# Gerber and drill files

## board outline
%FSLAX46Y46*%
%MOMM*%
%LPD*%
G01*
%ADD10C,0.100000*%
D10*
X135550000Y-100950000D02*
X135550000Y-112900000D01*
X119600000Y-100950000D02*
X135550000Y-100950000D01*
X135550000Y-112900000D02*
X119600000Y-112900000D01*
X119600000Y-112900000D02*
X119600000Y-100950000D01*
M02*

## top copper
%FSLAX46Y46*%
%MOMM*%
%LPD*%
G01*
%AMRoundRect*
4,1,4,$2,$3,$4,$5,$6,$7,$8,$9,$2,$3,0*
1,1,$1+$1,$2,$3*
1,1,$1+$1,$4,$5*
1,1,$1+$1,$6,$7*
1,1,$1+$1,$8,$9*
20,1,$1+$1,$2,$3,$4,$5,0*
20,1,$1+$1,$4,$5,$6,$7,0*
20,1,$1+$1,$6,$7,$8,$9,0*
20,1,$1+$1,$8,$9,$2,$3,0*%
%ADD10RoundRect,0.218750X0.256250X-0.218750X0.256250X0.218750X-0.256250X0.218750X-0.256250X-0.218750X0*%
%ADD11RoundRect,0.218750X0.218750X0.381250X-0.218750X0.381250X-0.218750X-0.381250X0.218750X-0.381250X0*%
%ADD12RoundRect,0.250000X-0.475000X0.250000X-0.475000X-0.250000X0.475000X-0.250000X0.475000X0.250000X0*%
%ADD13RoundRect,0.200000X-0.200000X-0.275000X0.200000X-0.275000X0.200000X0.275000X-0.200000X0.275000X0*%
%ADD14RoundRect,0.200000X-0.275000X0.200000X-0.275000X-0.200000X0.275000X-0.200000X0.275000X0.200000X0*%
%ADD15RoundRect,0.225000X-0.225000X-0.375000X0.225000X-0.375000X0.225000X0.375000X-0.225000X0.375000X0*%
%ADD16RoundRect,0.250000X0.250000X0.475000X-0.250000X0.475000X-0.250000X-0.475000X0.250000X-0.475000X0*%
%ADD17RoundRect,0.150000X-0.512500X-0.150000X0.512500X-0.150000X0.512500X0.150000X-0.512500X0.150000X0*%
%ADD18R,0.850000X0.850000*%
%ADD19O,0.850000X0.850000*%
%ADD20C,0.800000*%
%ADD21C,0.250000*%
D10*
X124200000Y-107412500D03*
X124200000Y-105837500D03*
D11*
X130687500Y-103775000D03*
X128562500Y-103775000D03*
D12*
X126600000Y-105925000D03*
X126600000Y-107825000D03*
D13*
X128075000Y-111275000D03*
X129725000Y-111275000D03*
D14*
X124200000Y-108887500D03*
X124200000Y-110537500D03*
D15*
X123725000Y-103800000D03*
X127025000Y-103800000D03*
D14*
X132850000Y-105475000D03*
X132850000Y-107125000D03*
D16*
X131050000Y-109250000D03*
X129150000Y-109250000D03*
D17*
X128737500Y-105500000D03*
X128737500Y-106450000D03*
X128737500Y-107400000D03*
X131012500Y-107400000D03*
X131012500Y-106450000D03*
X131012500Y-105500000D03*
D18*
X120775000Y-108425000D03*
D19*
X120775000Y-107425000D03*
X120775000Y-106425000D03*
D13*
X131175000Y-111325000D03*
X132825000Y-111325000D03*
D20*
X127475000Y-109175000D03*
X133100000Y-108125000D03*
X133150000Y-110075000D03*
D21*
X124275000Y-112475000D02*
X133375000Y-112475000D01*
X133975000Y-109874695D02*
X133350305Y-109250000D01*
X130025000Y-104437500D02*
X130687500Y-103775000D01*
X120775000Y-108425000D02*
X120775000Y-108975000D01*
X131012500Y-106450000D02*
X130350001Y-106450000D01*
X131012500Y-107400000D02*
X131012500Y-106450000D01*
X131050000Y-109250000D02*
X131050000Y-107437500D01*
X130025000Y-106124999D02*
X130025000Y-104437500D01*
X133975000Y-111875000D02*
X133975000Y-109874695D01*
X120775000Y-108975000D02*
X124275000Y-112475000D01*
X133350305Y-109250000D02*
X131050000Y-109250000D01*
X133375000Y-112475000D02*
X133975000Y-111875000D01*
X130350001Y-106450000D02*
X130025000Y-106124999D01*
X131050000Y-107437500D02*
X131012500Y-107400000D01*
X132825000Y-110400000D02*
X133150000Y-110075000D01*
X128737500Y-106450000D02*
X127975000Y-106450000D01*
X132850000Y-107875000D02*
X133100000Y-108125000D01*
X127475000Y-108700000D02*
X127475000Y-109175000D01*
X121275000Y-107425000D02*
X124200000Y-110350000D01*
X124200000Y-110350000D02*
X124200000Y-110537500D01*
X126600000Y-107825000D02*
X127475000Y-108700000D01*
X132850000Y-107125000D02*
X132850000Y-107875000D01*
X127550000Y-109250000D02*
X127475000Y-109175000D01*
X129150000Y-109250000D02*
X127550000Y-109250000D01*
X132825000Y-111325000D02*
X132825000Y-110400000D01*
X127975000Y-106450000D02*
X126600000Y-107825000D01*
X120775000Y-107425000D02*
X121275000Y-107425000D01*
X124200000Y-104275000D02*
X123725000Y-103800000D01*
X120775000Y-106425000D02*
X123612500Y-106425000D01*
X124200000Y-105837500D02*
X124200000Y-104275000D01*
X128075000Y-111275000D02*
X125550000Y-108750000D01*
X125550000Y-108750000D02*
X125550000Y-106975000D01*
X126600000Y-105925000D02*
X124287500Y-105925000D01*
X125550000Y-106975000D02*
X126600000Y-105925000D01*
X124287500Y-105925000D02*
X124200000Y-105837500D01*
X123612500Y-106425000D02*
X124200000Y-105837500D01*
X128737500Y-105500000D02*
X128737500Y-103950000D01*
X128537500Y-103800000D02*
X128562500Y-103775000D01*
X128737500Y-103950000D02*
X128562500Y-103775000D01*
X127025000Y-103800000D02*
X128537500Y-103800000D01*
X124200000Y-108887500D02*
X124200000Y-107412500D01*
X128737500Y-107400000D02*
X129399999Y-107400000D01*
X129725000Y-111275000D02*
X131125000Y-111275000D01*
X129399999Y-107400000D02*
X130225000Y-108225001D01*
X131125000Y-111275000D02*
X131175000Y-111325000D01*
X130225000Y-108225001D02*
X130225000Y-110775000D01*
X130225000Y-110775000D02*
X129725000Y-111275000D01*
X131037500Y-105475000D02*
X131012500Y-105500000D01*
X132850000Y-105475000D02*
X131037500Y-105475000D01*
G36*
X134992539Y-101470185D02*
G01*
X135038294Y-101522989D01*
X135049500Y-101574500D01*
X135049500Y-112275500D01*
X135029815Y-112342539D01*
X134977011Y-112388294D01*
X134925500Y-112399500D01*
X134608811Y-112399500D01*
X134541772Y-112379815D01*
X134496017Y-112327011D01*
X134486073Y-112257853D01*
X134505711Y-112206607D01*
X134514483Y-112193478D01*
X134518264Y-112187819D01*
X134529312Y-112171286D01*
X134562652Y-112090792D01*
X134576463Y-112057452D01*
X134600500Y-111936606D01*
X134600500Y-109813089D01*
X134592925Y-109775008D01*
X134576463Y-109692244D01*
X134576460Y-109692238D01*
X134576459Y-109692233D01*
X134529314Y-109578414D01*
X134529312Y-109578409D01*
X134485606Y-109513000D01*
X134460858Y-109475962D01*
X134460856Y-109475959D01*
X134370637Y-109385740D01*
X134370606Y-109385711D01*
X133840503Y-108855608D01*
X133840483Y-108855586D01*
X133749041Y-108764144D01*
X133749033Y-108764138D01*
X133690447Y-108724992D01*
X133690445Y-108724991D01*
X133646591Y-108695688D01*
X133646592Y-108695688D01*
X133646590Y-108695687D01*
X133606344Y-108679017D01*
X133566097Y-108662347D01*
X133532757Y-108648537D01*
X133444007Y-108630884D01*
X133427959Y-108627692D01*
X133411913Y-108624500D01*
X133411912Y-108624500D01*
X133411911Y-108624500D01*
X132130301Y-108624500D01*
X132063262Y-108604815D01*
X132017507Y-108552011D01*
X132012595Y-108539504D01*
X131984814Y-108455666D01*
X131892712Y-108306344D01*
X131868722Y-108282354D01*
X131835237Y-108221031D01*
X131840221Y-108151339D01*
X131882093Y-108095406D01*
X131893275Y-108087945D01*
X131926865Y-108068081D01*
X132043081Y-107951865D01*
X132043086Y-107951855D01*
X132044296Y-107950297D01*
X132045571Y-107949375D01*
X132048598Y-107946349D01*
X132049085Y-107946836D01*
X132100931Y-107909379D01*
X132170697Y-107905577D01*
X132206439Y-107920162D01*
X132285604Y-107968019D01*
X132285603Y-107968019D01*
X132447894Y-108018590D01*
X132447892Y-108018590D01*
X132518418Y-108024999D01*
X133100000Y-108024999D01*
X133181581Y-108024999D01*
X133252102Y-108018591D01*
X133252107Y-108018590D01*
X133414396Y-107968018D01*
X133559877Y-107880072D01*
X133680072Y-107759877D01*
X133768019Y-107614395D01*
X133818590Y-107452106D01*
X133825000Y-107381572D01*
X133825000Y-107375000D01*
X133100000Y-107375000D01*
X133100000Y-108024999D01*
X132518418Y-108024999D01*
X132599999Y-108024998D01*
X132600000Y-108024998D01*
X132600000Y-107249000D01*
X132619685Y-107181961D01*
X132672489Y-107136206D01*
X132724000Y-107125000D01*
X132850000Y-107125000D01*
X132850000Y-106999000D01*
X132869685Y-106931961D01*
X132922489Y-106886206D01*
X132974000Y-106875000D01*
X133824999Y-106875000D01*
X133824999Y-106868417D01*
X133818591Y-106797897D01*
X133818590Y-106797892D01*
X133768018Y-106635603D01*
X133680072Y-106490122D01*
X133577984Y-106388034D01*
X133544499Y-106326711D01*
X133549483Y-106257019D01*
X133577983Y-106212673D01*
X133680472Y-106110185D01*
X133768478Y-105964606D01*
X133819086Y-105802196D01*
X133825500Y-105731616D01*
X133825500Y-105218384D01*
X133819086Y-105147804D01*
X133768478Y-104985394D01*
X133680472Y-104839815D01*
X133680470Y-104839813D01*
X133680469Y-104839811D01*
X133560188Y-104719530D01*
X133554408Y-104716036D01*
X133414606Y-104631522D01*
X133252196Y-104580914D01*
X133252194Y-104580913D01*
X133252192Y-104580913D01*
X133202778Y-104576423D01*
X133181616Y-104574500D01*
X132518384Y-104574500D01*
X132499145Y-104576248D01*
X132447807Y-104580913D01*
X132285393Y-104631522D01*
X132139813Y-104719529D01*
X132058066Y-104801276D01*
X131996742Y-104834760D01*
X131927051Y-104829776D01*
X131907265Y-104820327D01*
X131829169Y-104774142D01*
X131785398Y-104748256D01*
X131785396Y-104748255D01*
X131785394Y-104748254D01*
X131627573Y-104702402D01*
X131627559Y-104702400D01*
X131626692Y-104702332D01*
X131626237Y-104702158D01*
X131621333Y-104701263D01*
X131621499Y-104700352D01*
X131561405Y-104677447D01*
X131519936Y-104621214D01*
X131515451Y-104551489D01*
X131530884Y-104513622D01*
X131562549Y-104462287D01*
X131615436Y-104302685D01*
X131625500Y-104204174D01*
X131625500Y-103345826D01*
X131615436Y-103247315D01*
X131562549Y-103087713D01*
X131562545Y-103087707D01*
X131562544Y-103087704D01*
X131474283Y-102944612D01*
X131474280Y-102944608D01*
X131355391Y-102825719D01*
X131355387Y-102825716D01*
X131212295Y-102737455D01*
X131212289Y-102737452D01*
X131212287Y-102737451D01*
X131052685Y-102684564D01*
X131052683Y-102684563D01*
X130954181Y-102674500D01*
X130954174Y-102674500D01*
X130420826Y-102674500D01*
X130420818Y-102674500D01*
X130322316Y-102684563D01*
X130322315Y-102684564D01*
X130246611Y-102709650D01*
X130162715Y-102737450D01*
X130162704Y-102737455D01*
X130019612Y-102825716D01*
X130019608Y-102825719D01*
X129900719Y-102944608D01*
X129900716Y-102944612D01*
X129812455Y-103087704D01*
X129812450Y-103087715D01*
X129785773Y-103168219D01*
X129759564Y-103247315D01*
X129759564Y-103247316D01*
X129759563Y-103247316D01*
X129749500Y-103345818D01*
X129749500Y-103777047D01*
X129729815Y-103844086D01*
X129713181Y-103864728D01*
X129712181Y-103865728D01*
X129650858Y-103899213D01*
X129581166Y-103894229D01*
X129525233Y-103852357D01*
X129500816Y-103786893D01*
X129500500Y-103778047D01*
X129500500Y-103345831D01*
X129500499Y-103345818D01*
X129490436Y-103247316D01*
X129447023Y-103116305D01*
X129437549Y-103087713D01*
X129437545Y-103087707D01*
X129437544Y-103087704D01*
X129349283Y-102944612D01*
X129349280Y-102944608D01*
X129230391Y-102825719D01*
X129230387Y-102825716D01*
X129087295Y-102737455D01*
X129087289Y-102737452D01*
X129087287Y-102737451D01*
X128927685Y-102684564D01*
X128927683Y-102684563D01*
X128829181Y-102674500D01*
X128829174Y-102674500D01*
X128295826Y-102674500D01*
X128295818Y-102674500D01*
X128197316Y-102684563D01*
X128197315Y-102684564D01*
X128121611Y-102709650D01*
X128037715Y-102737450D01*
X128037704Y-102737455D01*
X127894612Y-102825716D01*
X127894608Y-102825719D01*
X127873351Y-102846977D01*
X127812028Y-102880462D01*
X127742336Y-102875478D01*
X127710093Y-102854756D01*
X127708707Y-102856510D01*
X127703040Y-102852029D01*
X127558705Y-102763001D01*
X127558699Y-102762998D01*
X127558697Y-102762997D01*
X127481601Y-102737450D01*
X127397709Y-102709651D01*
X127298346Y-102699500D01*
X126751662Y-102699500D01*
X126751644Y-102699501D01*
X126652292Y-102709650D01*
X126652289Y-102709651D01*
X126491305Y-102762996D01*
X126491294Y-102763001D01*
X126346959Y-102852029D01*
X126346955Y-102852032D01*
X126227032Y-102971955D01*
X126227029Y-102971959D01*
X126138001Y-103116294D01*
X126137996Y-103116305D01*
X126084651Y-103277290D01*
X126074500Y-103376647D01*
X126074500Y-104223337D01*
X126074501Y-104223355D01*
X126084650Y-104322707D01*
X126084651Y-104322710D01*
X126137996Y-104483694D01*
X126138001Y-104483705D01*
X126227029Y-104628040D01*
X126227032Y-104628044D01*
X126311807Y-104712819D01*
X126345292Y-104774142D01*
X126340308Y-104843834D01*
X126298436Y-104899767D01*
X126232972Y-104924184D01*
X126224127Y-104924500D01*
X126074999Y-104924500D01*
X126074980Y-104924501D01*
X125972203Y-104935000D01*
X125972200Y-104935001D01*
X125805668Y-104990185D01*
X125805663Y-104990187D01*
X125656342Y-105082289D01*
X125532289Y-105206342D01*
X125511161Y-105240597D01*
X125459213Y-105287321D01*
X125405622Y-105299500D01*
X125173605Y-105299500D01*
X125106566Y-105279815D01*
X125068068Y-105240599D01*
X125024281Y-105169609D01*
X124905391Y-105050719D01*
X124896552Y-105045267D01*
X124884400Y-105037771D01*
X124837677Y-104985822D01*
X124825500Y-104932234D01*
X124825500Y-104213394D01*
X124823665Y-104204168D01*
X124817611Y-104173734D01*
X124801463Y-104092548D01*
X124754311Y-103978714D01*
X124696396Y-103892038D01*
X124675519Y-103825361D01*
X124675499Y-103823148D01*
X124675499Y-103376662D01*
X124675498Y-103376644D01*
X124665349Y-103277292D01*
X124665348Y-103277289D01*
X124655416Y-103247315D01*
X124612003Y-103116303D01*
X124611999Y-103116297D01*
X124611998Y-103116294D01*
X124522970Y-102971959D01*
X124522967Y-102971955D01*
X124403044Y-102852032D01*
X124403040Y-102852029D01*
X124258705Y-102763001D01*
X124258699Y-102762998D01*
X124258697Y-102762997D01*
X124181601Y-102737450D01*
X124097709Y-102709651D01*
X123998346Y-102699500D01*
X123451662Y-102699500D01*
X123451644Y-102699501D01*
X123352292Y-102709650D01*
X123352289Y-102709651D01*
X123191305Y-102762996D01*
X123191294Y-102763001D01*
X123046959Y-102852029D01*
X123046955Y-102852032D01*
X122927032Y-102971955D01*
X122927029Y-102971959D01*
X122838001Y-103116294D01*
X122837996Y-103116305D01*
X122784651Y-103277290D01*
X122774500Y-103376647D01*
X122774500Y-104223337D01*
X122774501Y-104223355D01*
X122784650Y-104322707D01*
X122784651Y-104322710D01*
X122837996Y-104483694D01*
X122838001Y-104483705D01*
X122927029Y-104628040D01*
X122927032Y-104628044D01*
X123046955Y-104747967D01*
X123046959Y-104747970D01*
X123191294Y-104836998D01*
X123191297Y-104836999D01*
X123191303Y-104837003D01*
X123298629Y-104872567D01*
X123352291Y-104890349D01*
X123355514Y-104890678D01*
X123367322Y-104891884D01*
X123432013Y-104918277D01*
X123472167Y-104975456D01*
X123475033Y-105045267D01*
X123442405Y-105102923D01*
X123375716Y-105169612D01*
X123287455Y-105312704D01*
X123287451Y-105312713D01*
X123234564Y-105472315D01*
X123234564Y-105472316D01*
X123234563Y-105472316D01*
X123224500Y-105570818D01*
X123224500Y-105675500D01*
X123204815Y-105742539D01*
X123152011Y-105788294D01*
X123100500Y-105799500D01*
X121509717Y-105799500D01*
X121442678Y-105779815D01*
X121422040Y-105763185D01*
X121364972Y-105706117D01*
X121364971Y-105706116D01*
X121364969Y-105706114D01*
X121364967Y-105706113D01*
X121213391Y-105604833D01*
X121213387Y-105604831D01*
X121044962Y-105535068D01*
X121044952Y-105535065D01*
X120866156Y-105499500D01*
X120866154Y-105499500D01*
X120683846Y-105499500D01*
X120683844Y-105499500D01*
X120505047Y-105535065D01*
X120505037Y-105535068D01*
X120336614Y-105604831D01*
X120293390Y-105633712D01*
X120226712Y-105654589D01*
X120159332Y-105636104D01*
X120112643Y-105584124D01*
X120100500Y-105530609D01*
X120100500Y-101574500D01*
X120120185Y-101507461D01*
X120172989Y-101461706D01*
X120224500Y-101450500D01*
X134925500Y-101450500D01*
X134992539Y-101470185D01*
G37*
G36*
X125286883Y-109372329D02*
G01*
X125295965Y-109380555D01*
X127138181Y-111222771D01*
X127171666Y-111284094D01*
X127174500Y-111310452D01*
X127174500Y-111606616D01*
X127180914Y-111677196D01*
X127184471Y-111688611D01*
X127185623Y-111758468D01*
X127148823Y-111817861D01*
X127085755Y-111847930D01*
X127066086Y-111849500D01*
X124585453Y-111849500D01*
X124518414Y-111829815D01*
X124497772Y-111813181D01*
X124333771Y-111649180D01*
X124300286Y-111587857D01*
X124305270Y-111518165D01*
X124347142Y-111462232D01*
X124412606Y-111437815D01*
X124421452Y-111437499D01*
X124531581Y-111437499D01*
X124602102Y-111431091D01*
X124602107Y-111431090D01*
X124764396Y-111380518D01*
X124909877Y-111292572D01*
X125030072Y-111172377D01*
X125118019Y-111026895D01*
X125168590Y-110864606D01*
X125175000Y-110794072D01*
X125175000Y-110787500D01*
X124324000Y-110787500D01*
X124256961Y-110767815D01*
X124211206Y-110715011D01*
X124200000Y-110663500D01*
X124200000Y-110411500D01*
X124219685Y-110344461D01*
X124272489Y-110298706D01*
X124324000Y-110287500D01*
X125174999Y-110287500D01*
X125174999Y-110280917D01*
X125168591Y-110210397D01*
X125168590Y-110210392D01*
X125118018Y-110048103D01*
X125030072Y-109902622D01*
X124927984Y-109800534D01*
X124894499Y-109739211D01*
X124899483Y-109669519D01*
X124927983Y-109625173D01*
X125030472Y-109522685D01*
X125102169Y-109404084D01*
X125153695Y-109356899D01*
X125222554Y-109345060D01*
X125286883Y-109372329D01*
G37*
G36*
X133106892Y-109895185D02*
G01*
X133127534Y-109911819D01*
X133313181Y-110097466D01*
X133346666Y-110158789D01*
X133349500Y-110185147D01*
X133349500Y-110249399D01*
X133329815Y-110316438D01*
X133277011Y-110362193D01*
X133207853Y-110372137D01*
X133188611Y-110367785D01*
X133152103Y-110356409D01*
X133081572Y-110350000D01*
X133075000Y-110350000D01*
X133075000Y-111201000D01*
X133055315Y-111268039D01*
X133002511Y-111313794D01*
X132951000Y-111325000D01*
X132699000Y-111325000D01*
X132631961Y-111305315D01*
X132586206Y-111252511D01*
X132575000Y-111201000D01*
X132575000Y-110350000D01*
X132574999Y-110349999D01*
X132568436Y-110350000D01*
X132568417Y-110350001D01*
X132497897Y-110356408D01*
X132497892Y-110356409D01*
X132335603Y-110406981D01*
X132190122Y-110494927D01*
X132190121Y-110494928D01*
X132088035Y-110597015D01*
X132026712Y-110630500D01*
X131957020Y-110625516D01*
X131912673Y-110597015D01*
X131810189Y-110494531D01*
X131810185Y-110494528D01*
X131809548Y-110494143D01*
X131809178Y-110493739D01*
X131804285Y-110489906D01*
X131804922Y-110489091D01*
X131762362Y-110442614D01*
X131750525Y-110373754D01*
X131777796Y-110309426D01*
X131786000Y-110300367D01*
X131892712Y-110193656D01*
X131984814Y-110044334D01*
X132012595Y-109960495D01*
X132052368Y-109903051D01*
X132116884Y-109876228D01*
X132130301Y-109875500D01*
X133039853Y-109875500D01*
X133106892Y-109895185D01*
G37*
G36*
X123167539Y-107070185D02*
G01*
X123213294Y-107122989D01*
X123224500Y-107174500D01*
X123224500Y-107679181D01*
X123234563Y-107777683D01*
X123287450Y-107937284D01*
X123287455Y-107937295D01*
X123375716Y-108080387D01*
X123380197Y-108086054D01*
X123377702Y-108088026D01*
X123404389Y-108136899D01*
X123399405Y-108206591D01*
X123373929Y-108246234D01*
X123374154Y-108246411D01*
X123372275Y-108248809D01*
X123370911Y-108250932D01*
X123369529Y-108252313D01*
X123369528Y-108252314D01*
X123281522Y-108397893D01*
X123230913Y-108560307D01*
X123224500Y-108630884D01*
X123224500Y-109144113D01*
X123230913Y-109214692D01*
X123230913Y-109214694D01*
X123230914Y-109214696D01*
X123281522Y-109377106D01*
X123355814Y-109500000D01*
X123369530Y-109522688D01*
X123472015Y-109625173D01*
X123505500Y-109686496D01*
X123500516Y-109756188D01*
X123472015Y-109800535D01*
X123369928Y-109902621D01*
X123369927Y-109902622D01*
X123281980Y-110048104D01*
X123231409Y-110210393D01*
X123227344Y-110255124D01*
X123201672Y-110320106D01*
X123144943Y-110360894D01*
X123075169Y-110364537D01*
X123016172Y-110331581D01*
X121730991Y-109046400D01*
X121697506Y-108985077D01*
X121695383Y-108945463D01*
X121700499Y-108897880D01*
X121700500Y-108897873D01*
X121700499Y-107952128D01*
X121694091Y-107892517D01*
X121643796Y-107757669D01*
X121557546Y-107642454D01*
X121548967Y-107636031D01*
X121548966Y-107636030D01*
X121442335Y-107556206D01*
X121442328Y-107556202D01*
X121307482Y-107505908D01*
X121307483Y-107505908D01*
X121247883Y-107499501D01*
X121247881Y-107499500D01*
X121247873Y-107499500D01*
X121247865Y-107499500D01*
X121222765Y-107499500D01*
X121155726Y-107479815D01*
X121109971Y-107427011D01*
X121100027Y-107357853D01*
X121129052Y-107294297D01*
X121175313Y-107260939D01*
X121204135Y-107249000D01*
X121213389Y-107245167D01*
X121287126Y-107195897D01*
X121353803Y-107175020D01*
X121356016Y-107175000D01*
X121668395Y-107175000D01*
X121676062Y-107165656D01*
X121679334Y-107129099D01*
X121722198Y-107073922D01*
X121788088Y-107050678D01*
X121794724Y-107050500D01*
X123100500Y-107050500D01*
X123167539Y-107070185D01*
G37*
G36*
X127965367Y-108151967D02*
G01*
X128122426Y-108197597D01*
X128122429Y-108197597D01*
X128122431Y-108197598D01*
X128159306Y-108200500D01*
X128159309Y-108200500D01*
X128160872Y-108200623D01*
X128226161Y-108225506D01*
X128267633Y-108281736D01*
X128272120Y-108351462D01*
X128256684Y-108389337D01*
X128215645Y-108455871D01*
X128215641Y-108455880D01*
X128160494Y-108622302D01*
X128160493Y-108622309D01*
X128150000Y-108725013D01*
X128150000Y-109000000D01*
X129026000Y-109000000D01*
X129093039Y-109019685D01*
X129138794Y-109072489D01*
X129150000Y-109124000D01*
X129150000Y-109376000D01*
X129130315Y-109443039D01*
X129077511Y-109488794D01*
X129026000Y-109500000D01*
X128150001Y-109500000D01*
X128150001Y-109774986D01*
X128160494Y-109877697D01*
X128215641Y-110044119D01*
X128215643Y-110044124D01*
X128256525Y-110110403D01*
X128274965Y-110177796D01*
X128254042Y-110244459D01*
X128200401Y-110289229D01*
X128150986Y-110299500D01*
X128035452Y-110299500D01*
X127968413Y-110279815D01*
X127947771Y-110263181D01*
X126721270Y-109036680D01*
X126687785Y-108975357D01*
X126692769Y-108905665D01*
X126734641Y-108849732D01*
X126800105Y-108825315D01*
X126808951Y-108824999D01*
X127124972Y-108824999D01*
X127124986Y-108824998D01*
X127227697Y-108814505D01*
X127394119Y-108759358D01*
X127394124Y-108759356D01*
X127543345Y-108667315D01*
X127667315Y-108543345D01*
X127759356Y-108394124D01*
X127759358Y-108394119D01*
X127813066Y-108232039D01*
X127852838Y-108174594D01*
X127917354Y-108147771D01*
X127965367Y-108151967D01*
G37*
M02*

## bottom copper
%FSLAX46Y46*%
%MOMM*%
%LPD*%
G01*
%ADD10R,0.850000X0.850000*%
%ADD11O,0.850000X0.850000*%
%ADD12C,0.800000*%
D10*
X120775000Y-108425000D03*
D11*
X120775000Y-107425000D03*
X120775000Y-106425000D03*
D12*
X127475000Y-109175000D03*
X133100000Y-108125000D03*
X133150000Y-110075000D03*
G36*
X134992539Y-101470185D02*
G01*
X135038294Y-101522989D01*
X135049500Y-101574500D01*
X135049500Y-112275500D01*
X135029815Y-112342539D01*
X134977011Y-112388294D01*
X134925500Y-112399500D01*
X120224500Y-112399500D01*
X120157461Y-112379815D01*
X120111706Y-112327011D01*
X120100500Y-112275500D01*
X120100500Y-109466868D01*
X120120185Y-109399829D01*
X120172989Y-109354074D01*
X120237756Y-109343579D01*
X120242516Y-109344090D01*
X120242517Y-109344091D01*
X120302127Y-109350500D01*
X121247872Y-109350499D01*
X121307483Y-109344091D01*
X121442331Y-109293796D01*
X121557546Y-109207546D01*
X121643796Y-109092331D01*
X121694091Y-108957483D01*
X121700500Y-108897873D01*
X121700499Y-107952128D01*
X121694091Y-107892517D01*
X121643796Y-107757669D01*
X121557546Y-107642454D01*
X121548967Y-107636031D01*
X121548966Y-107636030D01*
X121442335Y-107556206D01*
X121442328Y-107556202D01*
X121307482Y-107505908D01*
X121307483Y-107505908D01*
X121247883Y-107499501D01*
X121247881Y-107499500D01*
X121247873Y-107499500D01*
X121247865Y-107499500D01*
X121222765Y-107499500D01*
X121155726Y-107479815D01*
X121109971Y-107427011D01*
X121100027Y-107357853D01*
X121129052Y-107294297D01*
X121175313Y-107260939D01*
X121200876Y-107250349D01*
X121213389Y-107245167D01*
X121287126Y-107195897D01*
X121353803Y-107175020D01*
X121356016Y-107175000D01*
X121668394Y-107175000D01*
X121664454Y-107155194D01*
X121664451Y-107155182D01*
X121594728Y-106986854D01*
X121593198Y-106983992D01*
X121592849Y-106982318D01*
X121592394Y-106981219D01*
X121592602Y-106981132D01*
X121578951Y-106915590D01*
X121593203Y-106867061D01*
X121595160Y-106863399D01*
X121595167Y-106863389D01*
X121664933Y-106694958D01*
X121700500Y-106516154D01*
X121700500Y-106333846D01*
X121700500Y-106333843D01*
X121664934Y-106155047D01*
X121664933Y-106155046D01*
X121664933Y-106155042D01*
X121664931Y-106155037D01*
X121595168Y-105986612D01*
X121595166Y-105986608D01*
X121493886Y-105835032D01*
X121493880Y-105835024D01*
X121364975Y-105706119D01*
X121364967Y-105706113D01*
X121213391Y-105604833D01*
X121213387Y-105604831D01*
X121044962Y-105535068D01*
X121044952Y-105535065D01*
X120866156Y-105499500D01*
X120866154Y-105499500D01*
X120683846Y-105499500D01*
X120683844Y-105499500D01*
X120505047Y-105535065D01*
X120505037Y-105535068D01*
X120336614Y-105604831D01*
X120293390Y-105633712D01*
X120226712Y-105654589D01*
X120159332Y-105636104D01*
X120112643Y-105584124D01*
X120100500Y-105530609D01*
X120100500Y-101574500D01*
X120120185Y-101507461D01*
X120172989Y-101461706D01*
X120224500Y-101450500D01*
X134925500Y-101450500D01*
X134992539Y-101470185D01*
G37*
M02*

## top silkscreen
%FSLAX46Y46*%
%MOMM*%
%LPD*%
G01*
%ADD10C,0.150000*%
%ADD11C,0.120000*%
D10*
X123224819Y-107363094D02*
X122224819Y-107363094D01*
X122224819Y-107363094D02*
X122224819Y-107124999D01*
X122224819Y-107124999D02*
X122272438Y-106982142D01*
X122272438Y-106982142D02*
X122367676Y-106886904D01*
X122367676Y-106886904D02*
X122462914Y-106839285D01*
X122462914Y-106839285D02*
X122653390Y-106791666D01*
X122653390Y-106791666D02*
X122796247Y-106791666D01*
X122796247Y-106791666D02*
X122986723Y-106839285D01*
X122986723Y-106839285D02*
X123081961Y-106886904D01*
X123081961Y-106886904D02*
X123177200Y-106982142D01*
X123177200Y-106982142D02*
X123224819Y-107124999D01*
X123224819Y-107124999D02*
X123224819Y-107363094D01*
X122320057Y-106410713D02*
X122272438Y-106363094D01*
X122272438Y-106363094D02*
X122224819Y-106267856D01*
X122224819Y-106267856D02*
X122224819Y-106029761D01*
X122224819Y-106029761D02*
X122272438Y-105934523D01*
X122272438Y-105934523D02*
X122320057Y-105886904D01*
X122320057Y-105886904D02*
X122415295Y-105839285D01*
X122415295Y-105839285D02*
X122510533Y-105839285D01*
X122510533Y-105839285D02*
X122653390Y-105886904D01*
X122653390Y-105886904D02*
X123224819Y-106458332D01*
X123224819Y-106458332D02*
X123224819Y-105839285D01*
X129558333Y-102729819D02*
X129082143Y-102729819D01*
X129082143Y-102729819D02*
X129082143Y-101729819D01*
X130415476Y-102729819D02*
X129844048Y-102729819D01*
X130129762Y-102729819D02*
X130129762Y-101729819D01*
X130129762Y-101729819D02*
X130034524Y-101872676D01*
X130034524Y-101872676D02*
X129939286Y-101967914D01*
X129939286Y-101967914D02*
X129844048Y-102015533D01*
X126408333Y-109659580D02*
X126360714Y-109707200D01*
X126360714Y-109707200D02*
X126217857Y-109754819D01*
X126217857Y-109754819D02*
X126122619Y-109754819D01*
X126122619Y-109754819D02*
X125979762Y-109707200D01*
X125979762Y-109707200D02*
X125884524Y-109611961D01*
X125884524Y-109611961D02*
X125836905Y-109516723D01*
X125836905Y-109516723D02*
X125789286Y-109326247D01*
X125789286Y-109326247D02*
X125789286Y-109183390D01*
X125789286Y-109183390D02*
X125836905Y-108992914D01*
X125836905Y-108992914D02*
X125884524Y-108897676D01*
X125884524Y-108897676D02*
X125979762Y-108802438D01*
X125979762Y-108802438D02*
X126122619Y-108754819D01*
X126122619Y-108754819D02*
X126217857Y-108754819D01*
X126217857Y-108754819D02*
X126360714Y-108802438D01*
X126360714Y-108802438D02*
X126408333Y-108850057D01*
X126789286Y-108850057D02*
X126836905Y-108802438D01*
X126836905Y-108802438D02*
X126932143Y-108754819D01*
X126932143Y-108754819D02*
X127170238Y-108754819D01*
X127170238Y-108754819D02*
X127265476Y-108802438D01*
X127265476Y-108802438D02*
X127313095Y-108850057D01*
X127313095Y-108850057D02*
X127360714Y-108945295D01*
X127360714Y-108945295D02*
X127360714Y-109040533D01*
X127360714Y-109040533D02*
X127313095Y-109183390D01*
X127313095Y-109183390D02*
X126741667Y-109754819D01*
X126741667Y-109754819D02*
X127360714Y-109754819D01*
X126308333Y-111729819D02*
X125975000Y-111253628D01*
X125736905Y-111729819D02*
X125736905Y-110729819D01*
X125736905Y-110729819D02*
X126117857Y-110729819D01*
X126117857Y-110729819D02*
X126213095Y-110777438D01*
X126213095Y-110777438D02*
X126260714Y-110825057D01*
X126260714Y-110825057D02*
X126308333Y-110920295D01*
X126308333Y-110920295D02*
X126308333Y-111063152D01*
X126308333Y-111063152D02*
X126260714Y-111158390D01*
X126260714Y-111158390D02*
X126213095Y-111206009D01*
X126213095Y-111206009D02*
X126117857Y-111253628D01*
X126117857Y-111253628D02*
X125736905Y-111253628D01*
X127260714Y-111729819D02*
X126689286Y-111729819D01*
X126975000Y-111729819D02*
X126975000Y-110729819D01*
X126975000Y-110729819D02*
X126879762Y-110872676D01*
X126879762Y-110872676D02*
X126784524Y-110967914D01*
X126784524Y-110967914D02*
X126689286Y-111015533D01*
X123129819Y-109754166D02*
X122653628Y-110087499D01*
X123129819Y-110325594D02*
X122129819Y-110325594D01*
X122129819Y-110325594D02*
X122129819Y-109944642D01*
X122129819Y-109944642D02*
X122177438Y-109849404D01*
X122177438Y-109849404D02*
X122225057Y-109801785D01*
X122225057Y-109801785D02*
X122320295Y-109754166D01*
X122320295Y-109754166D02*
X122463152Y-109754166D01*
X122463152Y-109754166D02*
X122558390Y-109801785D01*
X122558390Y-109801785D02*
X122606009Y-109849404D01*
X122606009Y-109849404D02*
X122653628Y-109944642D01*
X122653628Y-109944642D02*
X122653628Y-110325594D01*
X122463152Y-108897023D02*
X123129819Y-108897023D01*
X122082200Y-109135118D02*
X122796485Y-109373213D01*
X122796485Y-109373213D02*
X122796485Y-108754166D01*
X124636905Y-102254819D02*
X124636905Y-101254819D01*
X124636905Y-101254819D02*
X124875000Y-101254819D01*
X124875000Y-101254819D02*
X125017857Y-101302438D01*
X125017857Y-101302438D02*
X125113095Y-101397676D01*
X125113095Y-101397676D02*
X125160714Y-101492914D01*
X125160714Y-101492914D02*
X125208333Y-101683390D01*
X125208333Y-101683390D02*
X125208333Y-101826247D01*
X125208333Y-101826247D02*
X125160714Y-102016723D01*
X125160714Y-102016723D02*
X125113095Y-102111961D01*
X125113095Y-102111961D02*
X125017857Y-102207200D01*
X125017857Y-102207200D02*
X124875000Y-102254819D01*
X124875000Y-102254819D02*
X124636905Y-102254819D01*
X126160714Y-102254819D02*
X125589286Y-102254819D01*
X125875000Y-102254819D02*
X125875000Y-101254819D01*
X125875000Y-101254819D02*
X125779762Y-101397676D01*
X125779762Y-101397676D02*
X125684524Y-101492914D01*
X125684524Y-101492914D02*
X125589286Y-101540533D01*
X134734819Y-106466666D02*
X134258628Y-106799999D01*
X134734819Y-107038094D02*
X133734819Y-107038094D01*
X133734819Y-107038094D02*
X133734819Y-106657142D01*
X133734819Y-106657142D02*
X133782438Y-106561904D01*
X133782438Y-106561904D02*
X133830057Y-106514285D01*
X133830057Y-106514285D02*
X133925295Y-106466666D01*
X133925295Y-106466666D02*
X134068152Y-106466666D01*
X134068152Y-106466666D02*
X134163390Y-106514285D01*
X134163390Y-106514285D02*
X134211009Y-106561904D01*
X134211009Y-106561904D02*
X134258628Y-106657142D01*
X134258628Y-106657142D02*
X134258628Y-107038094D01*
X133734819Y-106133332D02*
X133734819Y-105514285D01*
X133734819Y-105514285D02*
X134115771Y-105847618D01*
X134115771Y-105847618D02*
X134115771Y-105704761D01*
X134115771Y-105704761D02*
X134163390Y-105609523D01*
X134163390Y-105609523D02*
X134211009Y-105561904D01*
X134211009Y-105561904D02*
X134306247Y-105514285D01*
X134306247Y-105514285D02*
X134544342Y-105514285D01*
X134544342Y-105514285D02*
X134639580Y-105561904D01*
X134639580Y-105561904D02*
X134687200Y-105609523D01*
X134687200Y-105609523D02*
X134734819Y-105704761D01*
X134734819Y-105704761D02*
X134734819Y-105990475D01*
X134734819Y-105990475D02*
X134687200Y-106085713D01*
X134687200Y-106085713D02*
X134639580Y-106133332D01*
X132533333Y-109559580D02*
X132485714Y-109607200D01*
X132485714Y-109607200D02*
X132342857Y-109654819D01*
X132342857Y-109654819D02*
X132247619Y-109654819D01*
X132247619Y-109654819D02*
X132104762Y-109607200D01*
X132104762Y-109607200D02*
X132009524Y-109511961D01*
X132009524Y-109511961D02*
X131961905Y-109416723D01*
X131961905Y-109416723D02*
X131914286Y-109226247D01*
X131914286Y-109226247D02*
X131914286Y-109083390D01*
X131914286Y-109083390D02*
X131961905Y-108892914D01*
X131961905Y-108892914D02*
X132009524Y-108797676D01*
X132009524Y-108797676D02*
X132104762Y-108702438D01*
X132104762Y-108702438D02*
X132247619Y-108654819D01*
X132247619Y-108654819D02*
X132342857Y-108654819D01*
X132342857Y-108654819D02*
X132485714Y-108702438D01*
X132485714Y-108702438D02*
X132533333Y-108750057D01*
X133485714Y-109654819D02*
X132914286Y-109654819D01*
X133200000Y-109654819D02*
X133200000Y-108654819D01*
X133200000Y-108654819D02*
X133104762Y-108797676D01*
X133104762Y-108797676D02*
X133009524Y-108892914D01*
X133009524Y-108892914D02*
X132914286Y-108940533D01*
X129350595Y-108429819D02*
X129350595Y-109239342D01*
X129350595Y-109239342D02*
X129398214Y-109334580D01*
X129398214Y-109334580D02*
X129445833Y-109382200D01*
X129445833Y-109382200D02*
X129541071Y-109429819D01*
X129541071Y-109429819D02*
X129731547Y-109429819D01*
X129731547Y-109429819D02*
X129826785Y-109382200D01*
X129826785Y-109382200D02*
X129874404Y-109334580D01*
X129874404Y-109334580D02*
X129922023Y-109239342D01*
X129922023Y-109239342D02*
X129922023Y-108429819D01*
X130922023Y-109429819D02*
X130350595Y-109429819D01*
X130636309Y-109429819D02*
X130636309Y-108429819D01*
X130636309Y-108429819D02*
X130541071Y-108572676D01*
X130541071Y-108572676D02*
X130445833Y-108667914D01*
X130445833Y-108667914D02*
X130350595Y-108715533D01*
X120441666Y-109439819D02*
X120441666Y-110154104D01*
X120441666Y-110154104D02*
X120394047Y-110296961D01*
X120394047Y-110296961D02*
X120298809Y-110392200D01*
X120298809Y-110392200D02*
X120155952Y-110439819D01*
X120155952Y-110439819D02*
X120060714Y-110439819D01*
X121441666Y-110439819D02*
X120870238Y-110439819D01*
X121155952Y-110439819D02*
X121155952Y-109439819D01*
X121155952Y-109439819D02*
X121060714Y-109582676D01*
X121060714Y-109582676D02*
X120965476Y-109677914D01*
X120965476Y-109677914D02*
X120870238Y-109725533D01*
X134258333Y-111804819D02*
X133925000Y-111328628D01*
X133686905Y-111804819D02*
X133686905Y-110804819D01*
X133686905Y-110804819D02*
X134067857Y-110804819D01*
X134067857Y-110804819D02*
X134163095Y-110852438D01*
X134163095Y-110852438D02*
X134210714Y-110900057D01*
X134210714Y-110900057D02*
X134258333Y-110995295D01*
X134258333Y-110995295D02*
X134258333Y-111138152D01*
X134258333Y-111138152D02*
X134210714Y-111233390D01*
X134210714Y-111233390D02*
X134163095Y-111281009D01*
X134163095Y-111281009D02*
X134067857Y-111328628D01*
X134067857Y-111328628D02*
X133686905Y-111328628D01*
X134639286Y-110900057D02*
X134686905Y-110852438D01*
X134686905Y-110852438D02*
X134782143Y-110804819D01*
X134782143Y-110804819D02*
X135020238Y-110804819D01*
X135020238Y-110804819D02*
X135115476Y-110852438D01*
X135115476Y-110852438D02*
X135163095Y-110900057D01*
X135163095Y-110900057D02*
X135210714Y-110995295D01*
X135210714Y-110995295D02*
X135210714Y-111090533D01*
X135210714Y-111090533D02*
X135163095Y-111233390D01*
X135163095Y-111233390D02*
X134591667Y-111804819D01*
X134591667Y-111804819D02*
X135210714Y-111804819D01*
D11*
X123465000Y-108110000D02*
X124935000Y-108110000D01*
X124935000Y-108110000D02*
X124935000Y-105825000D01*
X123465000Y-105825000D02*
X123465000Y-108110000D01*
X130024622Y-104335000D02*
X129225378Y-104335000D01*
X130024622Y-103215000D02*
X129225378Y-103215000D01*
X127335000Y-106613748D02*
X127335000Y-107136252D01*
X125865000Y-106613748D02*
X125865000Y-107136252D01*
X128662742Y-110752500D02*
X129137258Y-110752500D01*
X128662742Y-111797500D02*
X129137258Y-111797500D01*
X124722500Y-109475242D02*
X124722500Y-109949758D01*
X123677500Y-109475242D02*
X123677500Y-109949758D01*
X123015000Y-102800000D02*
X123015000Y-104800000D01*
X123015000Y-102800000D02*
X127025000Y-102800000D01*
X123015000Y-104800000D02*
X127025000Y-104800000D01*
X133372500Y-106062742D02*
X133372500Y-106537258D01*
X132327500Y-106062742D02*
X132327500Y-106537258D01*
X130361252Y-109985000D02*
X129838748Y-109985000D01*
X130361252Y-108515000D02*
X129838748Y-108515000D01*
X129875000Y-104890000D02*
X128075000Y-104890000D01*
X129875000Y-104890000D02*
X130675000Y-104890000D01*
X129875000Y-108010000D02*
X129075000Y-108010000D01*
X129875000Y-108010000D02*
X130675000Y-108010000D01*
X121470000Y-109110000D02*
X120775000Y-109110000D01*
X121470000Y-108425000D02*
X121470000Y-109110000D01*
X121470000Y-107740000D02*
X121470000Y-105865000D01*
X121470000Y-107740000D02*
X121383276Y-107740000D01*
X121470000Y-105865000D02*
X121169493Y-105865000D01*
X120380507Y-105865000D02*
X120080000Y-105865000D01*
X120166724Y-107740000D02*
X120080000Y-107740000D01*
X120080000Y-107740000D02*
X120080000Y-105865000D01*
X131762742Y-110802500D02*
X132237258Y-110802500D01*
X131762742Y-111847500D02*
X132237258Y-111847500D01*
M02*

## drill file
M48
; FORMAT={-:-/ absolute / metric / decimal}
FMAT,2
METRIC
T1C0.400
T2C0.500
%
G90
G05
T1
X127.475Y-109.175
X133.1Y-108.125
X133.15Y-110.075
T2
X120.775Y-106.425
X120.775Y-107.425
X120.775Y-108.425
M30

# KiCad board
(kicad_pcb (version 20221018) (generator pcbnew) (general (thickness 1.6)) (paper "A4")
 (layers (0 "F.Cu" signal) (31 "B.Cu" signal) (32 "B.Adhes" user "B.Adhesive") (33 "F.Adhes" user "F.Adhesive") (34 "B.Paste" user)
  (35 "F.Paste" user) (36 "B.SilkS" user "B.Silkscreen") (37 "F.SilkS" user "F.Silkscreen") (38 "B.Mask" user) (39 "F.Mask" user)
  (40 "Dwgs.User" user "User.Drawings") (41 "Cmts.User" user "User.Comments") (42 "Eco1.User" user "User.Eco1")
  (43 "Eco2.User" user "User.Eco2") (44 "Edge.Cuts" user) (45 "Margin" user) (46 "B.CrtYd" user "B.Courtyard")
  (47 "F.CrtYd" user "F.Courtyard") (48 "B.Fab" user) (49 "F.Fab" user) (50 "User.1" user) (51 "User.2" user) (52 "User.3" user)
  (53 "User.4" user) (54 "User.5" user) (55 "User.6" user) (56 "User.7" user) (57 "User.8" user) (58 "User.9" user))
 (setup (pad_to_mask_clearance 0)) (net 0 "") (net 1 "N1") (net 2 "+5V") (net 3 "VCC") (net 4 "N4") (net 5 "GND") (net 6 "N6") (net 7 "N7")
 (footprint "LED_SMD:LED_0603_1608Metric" (layer "F.Cu") (at 124.2 106.625 90)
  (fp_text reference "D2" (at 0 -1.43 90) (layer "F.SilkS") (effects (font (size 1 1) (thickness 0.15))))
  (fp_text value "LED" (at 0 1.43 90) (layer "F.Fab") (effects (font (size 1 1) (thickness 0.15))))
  (fp_line (start -1.485 -0.735) (end -1.485 0.735) (stroke (width 0.12) (type solid)) (layer "F.SilkS"))
  (fp_line (start -1.485 0.735) (end 0.8 0.735) (stroke (width 0.12) (type solid)) (layer "F.SilkS"))
  (fp_line (start 0.8 -0.735) (end -1.485 -0.735) (stroke (width 0.12) (type solid)) (layer "F.SilkS"))
  (pad "1" smd roundrect (at -0.7875 0 90) (size 0.875 0.95) (layers "F.Cu" "F.Paste" "F.Mask") (roundrect_rratio 0.25) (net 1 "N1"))
  (pad "2" smd roundrect (at 0.7875 0 90) (size 0.875 0.95) (layers "F.Cu" "F.Paste" "F.Mask") (roundrect_rratio 0.25) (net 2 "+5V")))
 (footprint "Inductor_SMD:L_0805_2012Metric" (layer "F.Cu") (at 129.625 103.775 180)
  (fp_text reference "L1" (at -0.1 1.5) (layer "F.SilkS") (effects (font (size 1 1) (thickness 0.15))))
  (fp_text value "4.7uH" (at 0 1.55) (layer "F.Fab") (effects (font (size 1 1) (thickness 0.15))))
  (fp_line (start -0.399622 -0.56) (end 0.399622 -0.56) (stroke (width 0.12) (type solid)) (layer "F.SilkS"))
  (fp_line (start -0.399622 0.56) (end 0.399622 0.56) (stroke (width 0.12) (type solid)) (layer "F.SilkS"))
  (pad "1" smd roundrect (at -1.0625 0 180) (size 0.875 1.2) (layers "F.Cu" "F.Paste" "F.Mask") (roundrect_rratio 0.25) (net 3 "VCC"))
  (pad "2" smd roundrect (at 1.0625 0 180) (size 0.875 1.2) (layers "F.Cu" "F.Paste" "F.Mask") (roundrect_rratio 0.25) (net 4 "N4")))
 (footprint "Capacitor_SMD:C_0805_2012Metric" (layer "F.Cu") (at 126.6 106.875 -90)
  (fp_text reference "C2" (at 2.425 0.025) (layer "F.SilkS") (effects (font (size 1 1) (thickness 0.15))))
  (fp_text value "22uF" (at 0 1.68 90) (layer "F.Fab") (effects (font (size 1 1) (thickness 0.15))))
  (fp_line (start -0.261252 -0.735) (end 0.261252 -0.735) (stroke (width 0.12) (type solid)) (layer "F.SilkS"))
  (fp_line (start -0.261252 0.735) (end 0.261252 0.735) (stroke (width 0.12) (type solid)) (layer "F.SilkS"))
  (pad "1" smd roundrect (at -0.95 0 270) (size 1 1.45) (layers "F.Cu" "F.Paste" "F.Mask") (roundrect_rratio 0.25) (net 2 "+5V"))
  (pad "2" smd roundrect (at 0.95 0 270) (size 1 1.45) (layers "F.Cu" "F.Paste" "F.Mask") (roundrect_rratio 0.25) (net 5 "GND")))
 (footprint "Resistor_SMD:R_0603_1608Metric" (layer "F.Cu") (at 128.9 111.275)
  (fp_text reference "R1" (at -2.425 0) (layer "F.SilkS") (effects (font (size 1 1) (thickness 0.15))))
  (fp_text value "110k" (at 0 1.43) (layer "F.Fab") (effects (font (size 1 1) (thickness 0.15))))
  (fp_line (start -0.237258 -0.5225) (end 0.237258 -0.5225) (stroke (width 0.12) (type solid)) (layer "F.SilkS"))
  (fp_line (start -0.237258 0.5225) (end 0.237258 0.5225) (stroke (width 0.12) (type solid)) (layer "F.SilkS"))
  (pad "1" smd roundrect (at -0.825 0) (size 0.8 0.95) (layers "F.Cu" "F.Paste" "F.Mask") (roundrect_rratio 0.25) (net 2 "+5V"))
  (pad "2" smd roundrect (at 0.825 0) (size 0.8 0.95) (layers "F.Cu" "F.Paste" "F.Mask") (roundrect_rratio 0.25) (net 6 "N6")))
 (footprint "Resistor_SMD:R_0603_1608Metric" (layer "F.Cu") (at 124.2 109.7125 -90)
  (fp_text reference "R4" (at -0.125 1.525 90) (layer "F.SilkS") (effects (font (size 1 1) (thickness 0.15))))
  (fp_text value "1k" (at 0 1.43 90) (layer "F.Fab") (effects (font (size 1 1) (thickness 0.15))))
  (fp_line (start -0.237258 -0.5225) (end 0.237258 -0.5225) (stroke (width 0.12) (type solid)) (layer "F.SilkS"))
  (fp_line (start -0.237258 0.5225) (end 0.237258 0.5225) (stroke (width 0.12) (type solid)) (layer "F.SilkS"))
  (pad "1" smd roundrect (at -0.825 0 270) (size 0.8 0.95) (layers "F.Cu" "F.Paste" "F.Mask") (roundrect_rratio 0.25) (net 1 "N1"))
  (pad "2" smd roundrect (at 0.825 0 270) (size 0.8 0.95) (layers "F.Cu" "F.Paste" "F.Mask") (roundrect_rratio 0.25) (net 5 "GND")))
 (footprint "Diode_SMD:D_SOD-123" (layer "F.Cu") (at 125.375 103.8)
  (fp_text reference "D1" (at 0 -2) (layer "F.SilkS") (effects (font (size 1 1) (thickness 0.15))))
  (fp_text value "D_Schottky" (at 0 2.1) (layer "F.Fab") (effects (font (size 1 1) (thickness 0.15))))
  (fp_line (start -2.36 -1) (end -2.36 1) (stroke (width 0.12) (type solid)) (layer "F.SilkS"))
  (fp_line (start -2.36 -1) (end 1.65 -1) (stroke (width 0.12) (type solid)) (layer "F.SilkS"))
  (fp_line (start -2.36 1) (end 1.65 1) (stroke (width 0.12) (type solid)) (layer "F.SilkS"))
  (pad "1" smd roundrect (at -1.65 0) (size 0.9 1.2) (layers "F.Cu" "F.Paste" "F.Mask") (roundrect_rratio 0.25) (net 2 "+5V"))
  (pad "2" smd roundrect (at 1.65 0) (size 0.9 1.2) (layers "F.Cu" "F.Paste" "F.Mask") (roundrect_rratio 0.25) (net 4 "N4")))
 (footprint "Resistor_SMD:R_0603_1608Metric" (layer "F.Cu") (at 132.85 106.3 -90)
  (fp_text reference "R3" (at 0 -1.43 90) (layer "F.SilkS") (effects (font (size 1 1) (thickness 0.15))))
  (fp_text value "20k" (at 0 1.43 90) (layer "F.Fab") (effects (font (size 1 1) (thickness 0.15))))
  (fp_line (start -0.237258 -0.5225) (end 0.237258 -0.5225) (stroke (width 0.12) (type solid)) (layer "F.SilkS"))
  (fp_line (start -0.237258 0.5225) (end 0.237258 0.5225) (stroke (width 0.12) (type solid)) (layer "F.SilkS"))
  (pad "1" smd roundrect (at -0.825 0 270) (size 0.8 0.95) (layers "F.Cu" "F.Paste" "F.Mask") (roundrect_rratio 0.25) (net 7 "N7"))
  (pad "2" smd roundrect (at 0.825 0 270) (size 0.8 0.95) (layers "F.Cu" "F.Paste" "F.Mask") (roundrect_rratio 0.25) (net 5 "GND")))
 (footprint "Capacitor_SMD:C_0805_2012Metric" (layer "F.Cu") (at 130.1 109.25 180)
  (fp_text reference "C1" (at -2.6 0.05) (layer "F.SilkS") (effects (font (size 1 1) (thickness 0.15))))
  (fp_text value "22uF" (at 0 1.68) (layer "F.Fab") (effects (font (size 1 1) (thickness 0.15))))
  (fp_line (start -0.261252 -0.735) (end 0.261252 -0.735) (stroke (width 0.12) (type solid)) (layer "F.SilkS"))
  (fp_line (start -0.261252 0.735) (end 0.261252 0.735) (stroke (width 0.12) (type solid)) (layer "F.SilkS"))
  (pad "1" smd roundrect (at -0.95 0 180) (size 1 1.45) (layers "F.Cu" "F.Paste" "F.Mask") (roundrect_rratio 0.25) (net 3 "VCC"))
  (pad "2" smd roundrect (at 0.95 0 180) (size 1 1.45) (layers "F.Cu" "F.Paste" "F.Mask") (roundrect_rratio 0.25) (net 5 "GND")))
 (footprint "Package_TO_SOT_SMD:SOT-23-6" (layer "F.Cu") (at 129.875 106.45)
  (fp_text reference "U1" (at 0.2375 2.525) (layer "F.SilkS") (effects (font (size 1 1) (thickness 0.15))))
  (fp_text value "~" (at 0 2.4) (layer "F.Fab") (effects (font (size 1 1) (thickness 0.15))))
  (fp_line (start 0 -1.56) (end -1.8 -1.56) (stroke (width 0.12) (type solid)) (layer "F.SilkS"))
  (fp_line (start 0 -1.56) (end 0.8 -1.56) (stroke (width 0.12) (type solid)) (layer "F.SilkS"))
  (fp_line (start 0 1.56) (end -0.8 1.56) (stroke (width 0.12) (type solid)) (layer "F.SilkS"))
  (fp_line (start 0 1.56) (end 0.8 1.56) (stroke (width 0.12) (type solid)) (layer "F.SilkS"))
  (pad "1" smd roundrect (at -1.1375 -0.95) (size 1.325 0.6) (layers "F.Cu" "F.Paste" "F.Mask") (roundrect_rratio 0.25) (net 4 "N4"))
  (pad "2" smd roundrect (at -1.1375 0) (size 1.325 0.6) (layers "F.Cu" "F.Paste" "F.Mask") (roundrect_rratio 0.25) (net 5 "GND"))
  (pad "3" smd roundrect (at -1.1375 0.95) (size 1.325 0.6) (layers "F.Cu" "F.Paste" "F.Mask") (roundrect_rratio 0.25) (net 6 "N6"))
  (pad "4" smd roundrect (at 1.1375 0.95) (size 1.325 0.6) (layers "F.Cu" "F.Paste" "F.Mask") (roundrect_rratio 0.25) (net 3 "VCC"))
  (pad "5" smd roundrect (at 1.1375 0) (size 1.325 0.6) (layers "F.Cu" "F.Paste" "F.Mask") (roundrect_rratio 0.25) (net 3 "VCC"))
  (pad "6" smd roundrect (at 1.1375 -0.95) (size 1.325 0.6) (layers "F.Cu" "F.Paste" "F.Mask") (roundrect_rratio 0.25) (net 7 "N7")))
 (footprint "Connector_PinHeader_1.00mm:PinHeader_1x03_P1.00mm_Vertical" (layer "F.Cu") (at 120.775 108.425 180)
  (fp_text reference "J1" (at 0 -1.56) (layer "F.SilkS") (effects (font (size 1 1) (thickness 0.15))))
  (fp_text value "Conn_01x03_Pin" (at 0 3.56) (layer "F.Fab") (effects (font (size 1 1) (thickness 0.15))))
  (fp_line (start -0.695 -0.685) (end 0 -0.685) (stroke (width 0.12) (type solid)) (layer "F.SilkS"))
  (fp_line (start -0.695 0) (end -0.695 -0.685) (stroke (width 0.12) (type solid)) (layer "F.SilkS"))
  (fp_line (start -0.695 0.685) (end -0.695 2.56) (stroke (width 0.12) (type solid)) (layer "F.SilkS"))
  (fp_line (start -0.695 0.685) (end -0.608276 0.685) (stroke (width 0.12) (type solid)) (layer "F.SilkS"))
  (fp_line (start -0.695 2.56) (end -0.394493 2.56) (stroke (width 0.12) (type solid)) (layer "F.SilkS"))
  (fp_line (start 0.394493 2.56) (end 0.695 2.56) (stroke (width 0.12) (type solid)) (layer "F.SilkS"))
  (fp_line (start 0.608276 0.685) (end 0.695 0.685) (stroke (width 0.12) (type solid)) (layer "F.SilkS"))
  (fp_line (start 0.695 0.685) (end 0.695 2.56) (stroke (width 0.12) (type solid)) (layer "F.SilkS"))
  (pad "1" thru_hole rect (at 0 0 180) (size 0.85 0.85) (drill 0.5) (layers "*.Cu" "*.Mask") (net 3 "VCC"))
  (pad "2" thru_hole oval (at 0 1 180) (size 0.85 0.85) (drill 0.5) (layers "*.Cu" "*.Mask") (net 5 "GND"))
  (pad "3" thru_hole oval (at 0 2 180) (size 0.85 0.85) (drill 0.5) (layers "*.Cu" "*.Mask") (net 2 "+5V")))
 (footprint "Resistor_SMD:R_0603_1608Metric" (layer "F.Cu") (at 132 111.325)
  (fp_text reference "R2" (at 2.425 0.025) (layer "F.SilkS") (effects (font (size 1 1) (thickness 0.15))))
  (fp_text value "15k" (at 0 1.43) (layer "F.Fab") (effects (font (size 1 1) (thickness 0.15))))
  (fp_line (start -0.237258 -0.5225) (end 0.237258 -0.5225) (stroke (width 0.12) (type solid)) (layer "F.SilkS"))
  (fp_line (start -0.237258 0.5225) (end 0.237258 0.5225) (stroke (width 0.12) (type solid)) (layer "F.SilkS"))
  (pad "1" smd roundrect (at -0.825 0) (size 0.8 0.95) (layers "F.Cu" "F.Paste" "F.Mask") (roundrect_rratio 0.25) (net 6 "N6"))
  (pad "2" smd roundrect (at 0.825 0) (size 0.8 0.95) (layers "F.Cu" "F.Paste" "F.Mask") (roundrect_rratio 0.25) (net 5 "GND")))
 (gr_line (start 135.55 100.95) (end 135.55 112.9) (stroke (width 0.1) (type default)) (layer "Edge.Cuts"))
 (gr_line (start 119.6 100.95) (end 135.55 100.95) (stroke (width 0.1) (type default)) (layer "Edge.Cuts"))
 (gr_line (start 135.55 112.9) (end 119.6 112.9) (stroke (width 0.1) (type default)) (layer "Edge.Cuts"))
 (gr_line (start 119.6 112.9) (end 119.6 100.95) (stroke (width 0.1) (type default)) (layer "Edge.Cuts"))
 (segment (start 124.275 112.475) (end 133.375 112.475) (width 0.25) (layer "F.Cu") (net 3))
 (segment (start 133.975 109.874695) (end 133.350305 109.25) (width 0.25) (layer "F.Cu") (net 3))
 (segment (start 130.025 104.4375) (end 130.6875 103.775) (width 0.25) (layer "F.Cu") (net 3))
 (segment (start 120.775 108.425) (end 120.775 108.975) (width 0.25) (layer "F.Cu") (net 3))
 (segment (start 131.0125 106.45) (end 130.350001 106.45) (width 0.25) (layer "F.Cu") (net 3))
 (segment (start 131.0125 107.4) (end 131.0125 106.45) (width 0.25) (layer "F.Cu") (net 3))
 (segment (start 131.05 109.25) (end 131.05 107.4375) (width 0.25) (layer "F.Cu") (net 3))
 (segment (start 130.025 106.124999) (end 130.025 104.4375) (width 0.25) (layer "F.Cu") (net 3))
 (segment (start 133.975 111.875) (end 133.975 109.874695) (width 0.25) (layer "F.Cu") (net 3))
 (segment (start 120.775 108.975) (end 124.275 112.475) (width 0.25) (layer "F.Cu") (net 3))
 (segment (start 133.350305 109.25) (end 131.05 109.25) (width 0.25) (layer "F.Cu") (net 3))
 (segment (start 133.375 112.475) (end 133.975 111.875) (width 0.25) (layer "F.Cu") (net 3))
 (segment (start 130.350001 106.45) (end 130.025 106.124999) (width 0.25) (layer "F.Cu") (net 3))
 (segment (start 131.05 107.4375) (end 131.0125 107.4) (width 0.25) (layer "F.Cu") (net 3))
 (segment (start 132.825 110.4) (end 133.15 110.075) (width 0.25) (layer "F.Cu") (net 5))
 (segment (start 128.7375 106.45) (end 127.975 106.45) (width 0.25) (layer "F.Cu") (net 5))
 (segment (start 132.85 107.875) (end 133.1 108.125) (width 0.25) (layer "F.Cu") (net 5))
 (segment (start 127.475 108.7) (end 127.475 109.175) (width 0.25) (layer "F.Cu") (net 5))
 (segment (start 121.275 107.425) (end 124.2 110.35) (width 0.25) (layer "F.Cu") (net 5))
 (segment (start 124.2 110.35) (end 124.2 110.5375) (width 0.25) (layer "F.Cu") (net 5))
 (segment (start 126.6 107.825) (end 127.475 108.7) (width 0.25) (layer "F.Cu") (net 5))
 (segment (start 132.85 107.125) (end 132.85 107.875) (width 0.25) (layer "F.Cu") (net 5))
 (segment (start 127.55 109.25) (end 127.475 109.175) (width 0.25) (layer "F.Cu") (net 5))
 (segment (start 129.15 109.25) (end 127.55 109.25) (width 0.25) (layer "F.Cu") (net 5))
 (segment (start 132.825 111.325) (end 132.825 110.4) (width 0.25) (layer "F.Cu") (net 5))
 (segment (start 127.975 106.45) (end 126.6 107.825) (width 0.25) (layer "F.Cu") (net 5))
 (segment (start 120.775 107.425) (end 121.275 107.425) (width 0.25) (layer "F.Cu") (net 5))
 (via (at 127.475 109.175) (size 0.8) (drill 0.4) (layers "F.Cu" "B.Cu") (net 5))
 (via (at 133.1 108.125) (size 0.8) (drill 0.4) (layers "F.Cu" "B.Cu") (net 5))
 (via (at 133.15 110.075) (size 0.8) (drill 0.4) (layers "F.Cu" "B.Cu") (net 5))
 (segment (start 124.2 104.275) (end 123.725 103.8) (width 0.25) (layer "F.Cu") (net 2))
 (segment (start 120.775 106.425) (end 123.6125 106.425) (width 0.25) (layer "F.Cu") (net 2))
 (segment (start 124.2 105.8375) (end 124.2 104.275) (width 0.25) (layer "F.Cu") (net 2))
 (segment (start 128.075 111.275) (end 125.55 108.75) (width 0.25) (layer "F.Cu") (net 2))
 (segment (start 125.55 108.75) (end 125.55 106.975) (width 0.25) (layer "F.Cu") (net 2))
 (segment (start 126.6 105.925) (end 124.2875 105.925) (width 0.25) (layer "F.Cu") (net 2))
 (segment (start 125.55 106.975) (end 126.6 105.925) (width 0.25) (layer "F.Cu") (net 2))
 (segment (start 124.2875 105.925) (end 124.2 105.8375) (width 0.25) (layer "F.Cu") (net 2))
 (segment (start 123.6125 106.425) (end 124.2 105.8375) (width 0.25) (layer "F.Cu") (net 2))
 (segment (start 128.7375 105.5) (end 128.7375 103.95) (width 0.25) (layer "F.Cu") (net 4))
 (segment (start 128.5375 103.8) (end 128.5625 103.775) (width 0.25) (layer "F.Cu") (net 4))
 (segment (start 128.7375 103.95) (end 128.5625 103.775) (width 0.25) (layer "F.Cu") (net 4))
 (segment (start 127.025 103.8) (end 128.5375 103.8) (width 0.25) (layer "F.Cu") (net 4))
 (segment (start 124.2 108.8875) (end 124.2 107.4125) (width 0.25) (layer "F.Cu") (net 1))
 (segment (start 128.7375 107.4) (end 129.399999 107.4) (width 0.25) (layer "F.Cu") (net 6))
 (segment (start 129.725 111.275) (end 131.125 111.275) (width 0.25) (layer "F.Cu") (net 6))
 (segment (start 129.399999 107.4) (end 130.225 108.225001) (width 0.25) (layer "F.Cu") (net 6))
 (segment (start 131.125 111.275) (end 131.175 111.325) (width 0.25) (layer "F.Cu") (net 6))
 (segment (start 130.225 108.225001) (end 130.225 110.775) (width 0.25) (layer "F.Cu") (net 6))
 (segment (start 130.225 110.775) (end 129.725 111.275) (width 0.25) (layer "F.Cu") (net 6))
 (segment (start 131.0375 105.475) (end 131.0125 105.5) (width 0.25) (layer "F.Cu") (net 7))
 (segment (start 132.85 105.475) (end 131.0375 105.475) (width 0.25) (layer "F.Cu") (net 7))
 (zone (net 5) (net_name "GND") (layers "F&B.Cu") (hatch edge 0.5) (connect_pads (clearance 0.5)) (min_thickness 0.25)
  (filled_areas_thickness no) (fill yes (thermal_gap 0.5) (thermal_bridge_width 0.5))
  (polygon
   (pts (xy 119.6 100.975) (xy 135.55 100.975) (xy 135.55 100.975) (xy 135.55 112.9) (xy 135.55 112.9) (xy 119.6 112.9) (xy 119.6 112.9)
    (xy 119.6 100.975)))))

